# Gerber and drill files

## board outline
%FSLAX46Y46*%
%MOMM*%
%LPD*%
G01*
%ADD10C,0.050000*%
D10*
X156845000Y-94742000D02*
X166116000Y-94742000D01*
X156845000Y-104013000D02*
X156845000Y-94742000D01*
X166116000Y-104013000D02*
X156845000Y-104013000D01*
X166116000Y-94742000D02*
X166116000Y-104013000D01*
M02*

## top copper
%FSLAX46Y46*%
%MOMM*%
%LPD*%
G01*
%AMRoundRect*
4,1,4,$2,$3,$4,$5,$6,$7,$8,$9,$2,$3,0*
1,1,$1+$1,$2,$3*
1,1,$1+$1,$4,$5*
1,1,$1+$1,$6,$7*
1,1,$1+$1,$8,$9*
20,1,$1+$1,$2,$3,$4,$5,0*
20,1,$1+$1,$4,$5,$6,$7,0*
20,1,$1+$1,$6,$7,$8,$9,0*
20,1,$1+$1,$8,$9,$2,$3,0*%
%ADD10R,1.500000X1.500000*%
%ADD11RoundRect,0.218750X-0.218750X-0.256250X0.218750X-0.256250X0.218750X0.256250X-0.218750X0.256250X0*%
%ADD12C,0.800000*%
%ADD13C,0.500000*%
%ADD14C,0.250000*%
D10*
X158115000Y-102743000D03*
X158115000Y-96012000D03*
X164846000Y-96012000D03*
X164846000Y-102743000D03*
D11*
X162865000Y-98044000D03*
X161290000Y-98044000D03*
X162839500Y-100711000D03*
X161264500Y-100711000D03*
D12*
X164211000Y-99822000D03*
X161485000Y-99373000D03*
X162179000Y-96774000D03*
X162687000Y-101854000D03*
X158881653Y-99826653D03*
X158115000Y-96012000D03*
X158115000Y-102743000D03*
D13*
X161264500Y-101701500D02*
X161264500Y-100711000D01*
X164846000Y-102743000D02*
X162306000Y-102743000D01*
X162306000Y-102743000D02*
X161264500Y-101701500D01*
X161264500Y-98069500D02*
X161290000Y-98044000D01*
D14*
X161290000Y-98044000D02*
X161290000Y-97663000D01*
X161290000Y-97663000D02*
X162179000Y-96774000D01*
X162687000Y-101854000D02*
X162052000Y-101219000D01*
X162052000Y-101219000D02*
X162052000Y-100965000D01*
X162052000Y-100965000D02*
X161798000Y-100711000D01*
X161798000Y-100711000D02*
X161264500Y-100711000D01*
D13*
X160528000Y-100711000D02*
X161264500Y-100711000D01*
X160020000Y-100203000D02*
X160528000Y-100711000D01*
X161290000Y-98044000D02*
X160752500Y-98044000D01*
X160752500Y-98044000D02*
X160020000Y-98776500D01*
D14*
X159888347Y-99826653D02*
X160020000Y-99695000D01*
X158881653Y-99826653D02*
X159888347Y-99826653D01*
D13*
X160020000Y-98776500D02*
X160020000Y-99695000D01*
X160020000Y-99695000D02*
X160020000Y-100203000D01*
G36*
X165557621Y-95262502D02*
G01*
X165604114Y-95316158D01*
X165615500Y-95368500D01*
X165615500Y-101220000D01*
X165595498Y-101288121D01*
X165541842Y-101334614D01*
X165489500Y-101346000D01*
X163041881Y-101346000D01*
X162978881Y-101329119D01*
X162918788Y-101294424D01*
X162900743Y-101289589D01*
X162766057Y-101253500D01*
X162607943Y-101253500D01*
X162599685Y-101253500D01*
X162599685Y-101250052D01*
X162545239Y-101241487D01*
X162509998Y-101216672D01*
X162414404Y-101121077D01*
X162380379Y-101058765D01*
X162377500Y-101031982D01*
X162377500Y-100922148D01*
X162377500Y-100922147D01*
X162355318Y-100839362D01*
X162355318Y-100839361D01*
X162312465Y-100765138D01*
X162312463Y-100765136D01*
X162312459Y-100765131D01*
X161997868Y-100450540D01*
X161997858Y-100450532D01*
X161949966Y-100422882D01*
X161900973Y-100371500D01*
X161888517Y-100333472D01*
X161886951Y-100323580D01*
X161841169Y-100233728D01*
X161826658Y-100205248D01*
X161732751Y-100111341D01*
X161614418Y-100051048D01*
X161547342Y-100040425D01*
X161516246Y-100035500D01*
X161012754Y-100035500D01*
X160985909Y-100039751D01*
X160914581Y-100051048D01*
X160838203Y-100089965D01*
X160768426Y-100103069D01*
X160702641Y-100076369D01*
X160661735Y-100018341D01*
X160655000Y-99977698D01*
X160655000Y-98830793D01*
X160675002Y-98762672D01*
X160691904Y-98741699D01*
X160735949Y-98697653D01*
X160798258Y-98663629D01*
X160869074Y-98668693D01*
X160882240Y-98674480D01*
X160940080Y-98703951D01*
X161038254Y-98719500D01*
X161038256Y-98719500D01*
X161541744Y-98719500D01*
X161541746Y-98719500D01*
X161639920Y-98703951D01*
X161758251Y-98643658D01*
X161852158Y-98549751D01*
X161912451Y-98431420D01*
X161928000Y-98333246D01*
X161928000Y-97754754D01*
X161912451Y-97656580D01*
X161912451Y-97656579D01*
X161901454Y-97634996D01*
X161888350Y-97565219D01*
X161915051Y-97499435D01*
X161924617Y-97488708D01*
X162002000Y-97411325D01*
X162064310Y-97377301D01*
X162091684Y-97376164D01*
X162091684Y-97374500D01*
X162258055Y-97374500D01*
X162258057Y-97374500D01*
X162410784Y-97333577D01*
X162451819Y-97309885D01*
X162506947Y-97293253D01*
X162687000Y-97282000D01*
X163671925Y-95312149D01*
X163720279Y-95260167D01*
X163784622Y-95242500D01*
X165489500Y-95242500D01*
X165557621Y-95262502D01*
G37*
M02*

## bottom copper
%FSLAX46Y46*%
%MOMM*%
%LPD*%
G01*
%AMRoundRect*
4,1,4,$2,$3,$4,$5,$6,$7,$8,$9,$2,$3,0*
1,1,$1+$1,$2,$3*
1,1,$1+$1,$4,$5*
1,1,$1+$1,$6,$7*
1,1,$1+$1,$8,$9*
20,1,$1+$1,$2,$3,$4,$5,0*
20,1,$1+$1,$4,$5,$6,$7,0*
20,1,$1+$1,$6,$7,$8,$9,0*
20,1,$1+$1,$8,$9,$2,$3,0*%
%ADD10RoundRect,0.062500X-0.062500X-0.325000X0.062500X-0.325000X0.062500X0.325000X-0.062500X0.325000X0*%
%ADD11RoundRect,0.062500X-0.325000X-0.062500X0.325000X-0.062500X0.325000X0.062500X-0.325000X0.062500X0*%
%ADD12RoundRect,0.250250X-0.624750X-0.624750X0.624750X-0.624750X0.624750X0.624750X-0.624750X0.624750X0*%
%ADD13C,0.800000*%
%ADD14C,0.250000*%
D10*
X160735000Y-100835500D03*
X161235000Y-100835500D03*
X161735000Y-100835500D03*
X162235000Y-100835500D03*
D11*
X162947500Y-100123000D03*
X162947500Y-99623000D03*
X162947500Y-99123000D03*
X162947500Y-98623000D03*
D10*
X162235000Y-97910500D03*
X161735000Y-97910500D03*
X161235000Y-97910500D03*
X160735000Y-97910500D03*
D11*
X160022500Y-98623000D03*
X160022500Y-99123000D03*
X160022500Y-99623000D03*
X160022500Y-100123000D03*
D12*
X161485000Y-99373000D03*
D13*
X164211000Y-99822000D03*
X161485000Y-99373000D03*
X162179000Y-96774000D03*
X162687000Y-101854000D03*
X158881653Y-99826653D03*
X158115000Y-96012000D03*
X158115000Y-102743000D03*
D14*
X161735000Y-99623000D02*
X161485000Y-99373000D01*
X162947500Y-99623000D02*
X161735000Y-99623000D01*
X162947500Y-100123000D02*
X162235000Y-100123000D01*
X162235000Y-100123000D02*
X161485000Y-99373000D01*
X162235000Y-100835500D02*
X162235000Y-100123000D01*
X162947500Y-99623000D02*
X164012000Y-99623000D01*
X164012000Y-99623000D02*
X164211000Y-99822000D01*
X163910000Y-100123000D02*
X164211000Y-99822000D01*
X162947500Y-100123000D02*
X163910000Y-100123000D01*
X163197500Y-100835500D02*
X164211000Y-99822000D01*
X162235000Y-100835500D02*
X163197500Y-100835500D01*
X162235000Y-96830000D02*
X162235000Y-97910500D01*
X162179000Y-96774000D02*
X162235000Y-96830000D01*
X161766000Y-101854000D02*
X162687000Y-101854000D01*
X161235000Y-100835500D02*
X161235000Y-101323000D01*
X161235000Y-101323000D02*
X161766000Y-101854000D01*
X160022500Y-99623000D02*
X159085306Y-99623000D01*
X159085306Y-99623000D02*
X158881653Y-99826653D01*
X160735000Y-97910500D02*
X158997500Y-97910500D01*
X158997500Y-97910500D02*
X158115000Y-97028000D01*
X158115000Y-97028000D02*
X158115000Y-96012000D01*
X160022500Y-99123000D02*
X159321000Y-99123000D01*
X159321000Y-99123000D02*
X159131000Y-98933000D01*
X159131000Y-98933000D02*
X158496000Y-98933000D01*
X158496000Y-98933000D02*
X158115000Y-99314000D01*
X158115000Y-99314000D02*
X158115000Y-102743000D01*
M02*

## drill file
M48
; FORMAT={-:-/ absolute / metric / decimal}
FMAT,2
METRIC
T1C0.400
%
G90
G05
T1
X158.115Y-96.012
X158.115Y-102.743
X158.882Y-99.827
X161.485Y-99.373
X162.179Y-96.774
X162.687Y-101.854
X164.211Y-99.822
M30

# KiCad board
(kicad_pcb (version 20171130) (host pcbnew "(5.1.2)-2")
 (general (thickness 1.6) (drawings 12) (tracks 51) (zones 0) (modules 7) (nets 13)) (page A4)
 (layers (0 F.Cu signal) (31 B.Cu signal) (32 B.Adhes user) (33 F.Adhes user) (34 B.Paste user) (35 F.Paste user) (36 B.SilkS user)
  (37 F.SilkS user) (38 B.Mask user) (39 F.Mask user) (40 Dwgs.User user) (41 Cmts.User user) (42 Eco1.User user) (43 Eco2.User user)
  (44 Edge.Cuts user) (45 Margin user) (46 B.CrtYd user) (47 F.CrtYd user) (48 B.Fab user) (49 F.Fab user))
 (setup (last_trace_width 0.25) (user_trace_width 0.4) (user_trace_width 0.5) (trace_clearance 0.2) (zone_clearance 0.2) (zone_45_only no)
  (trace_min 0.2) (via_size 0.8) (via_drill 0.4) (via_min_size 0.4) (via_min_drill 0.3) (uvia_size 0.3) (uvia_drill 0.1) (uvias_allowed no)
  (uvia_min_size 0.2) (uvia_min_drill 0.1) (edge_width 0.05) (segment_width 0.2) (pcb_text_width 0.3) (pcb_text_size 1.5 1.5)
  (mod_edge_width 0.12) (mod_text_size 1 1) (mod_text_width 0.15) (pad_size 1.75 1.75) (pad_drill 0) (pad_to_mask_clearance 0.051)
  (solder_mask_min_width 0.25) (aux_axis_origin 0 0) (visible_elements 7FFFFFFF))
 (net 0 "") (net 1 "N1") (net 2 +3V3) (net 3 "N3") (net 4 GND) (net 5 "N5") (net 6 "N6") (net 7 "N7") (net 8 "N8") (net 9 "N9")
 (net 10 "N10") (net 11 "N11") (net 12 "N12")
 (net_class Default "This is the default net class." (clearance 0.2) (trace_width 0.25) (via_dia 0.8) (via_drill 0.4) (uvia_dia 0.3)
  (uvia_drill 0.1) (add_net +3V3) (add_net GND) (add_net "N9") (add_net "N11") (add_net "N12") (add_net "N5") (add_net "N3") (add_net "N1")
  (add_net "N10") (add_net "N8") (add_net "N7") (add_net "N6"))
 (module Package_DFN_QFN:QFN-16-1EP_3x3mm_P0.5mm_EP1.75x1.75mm (layer B.Cu) (at 161.485 99.373)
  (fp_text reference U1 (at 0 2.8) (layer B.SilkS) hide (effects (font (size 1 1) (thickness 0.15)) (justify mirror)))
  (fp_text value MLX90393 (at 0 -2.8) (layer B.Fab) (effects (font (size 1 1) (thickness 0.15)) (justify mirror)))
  (pad 16 smd roundrect (at -0.75 1.4625) (size 0.25 0.775) (layers B.Cu B.Paste B.Mask) (roundrect_rratio 0.25) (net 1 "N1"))
  (pad 15 smd roundrect (at -0.25 1.4625) (size 0.25 0.775) (layers B.Cu B.Paste B.Mask) (roundrect_rratio 0.25) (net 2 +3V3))
  (pad 14 smd roundrect (at 0.25 1.4625) (size 0.25 0.775) (layers B.Cu B.Paste B.Mask) (roundrect_rratio 0.25) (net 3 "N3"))
  (pad 13 smd roundrect (at 0.75 1.4625) (size 0.25 0.775) (layers B.Cu B.Paste B.Mask) (roundrect_rratio 0.25) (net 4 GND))
  (pad 12 smd roundrect (at 1.4625 0.75) (size 0.775 0.25) (layers B.Cu B.Paste B.Mask) (roundrect_rratio 0.25) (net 4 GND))
  (pad 11 smd roundrect (at 1.4625 0.25) (size 0.775 0.25) (layers B.Cu B.Paste B.Mask) (roundrect_rratio 0.25) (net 4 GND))
  (pad 10 smd roundrect (at 1.4625 -0.25) (size 0.775 0.25) (layers B.Cu B.Paste B.Mask) (roundrect_rratio 0.25) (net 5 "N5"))
  (pad 9 smd roundrect (at 1.4625 -0.75) (size 0.775 0.25) (layers B.Cu B.Paste B.Mask) (roundrect_rratio 0.25) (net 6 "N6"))
  (pad 8 smd roundrect (at 0.75 -1.4625) (size 0.25 0.775) (layers B.Cu B.Paste B.Mask) (roundrect_rratio 0.25) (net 2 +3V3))
  (pad 7 smd roundrect (at 0.25 -1.4625) (size 0.25 0.775) (layers B.Cu B.Paste B.Mask) (roundrect_rratio 0.25) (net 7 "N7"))
  (pad 6 smd roundrect (at -0.25 -1.4625) (size 0.25 0.775) (layers B.Cu B.Paste B.Mask) (roundrect_rratio 0.25) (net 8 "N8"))
  (pad 5 smd roundrect (at -0.75 -1.4625) (size 0.25 0.775) (layers B.Cu B.Paste B.Mask) (roundrect_rratio 0.25) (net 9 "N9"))
  (pad 4 smd roundrect (at -1.4625 -0.75) (size 0.775 0.25) (layers B.Cu B.Paste B.Mask) (roundrect_rratio 0.25) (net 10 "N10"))
  (pad 3 smd roundrect (at -1.4625 -0.25) (size 0.775 0.25) (layers B.Cu B.Paste B.Mask) (roundrect_rratio 0.25) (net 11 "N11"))
  (pad 2 smd roundrect (at -1.4625 0.25) (size 0.775 0.25) (layers B.Cu B.Paste B.Mask) (roundrect_rratio 0.25) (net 2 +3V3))
  (pad 1 smd roundrect (at -1.4625 0.75) (size 0.775 0.25) (layers B.Cu B.Paste B.Mask) (roundrect_rratio 0.25) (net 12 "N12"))
  (pad "" smd roundrect (at 0.44 -0.44) (size 0.71 0.71) (layers B.Paste) (roundrect_rratio 0.25))
  (pad "" smd roundrect (at 0.44 0.44) (size 0.71 0.71) (layers B.Paste) (roundrect_rratio 0.25))
  (pad "" smd roundrect (at -0.44 -0.44) (size 0.71 0.71) (layers B.Paste) (roundrect_rratio 0.25))
  (pad "" smd roundrect (at -0.44 0.44) (size 0.71 0.71) (layers B.Paste) (roundrect_rratio 0.25))
  (pad 17 smd roundrect (at 0 0) (size 1.75 1.75) (layers B.Cu B.Mask) (roundrect_rratio 0.143) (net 4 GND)))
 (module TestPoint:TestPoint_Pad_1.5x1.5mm (layer F.Cu) (at 158.115 102.743)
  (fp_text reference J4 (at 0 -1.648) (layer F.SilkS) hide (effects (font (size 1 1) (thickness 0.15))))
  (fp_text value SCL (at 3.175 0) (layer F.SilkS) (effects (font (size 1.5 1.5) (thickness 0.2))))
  (pad 1 smd rect (at 0 0) (size 1.5 1.5) (layers F.Cu F.Mask) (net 11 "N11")))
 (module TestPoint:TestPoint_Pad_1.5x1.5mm (layer F.Cu) (at 158.115 96.012)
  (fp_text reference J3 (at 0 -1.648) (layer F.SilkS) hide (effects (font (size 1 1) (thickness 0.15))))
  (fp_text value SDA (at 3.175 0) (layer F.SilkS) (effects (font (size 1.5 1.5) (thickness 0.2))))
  (pad 1 smd rect (at 0 0) (size 1.5 1.5) (layers F.Cu F.Mask) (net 9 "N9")))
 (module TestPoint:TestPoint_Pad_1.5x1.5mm (layer F.Cu) (at 164.846 96.012)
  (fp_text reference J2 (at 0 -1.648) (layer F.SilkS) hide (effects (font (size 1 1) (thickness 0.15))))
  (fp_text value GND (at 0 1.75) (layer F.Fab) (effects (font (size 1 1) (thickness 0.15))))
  (pad 1 smd rect (at 0 0) (size 1.5 1.5) (layers F.Cu F.Mask) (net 4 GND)))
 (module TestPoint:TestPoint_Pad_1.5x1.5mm (layer F.Cu) (at 164.846 102.743)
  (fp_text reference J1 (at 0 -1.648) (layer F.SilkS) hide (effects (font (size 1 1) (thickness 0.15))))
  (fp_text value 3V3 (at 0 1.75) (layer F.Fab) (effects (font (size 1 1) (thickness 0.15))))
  (pad 1 smd rect (at 0 0) (size 1.5 1.5) (layers F.Cu F.Mask) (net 2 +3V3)))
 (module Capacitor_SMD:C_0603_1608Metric (layer F.Cu) (at 162.0775 98.044)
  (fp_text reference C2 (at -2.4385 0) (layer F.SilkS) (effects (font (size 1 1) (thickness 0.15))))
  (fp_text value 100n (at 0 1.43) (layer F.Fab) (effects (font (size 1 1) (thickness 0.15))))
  (pad 2 smd roundrect (at 0.7875 0) (size 0.875 0.95) (layers F.Cu F.Paste F.Mask) (roundrect_rratio 0.25) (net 4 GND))
  (pad 1 smd roundrect (at -0.7875 0) (size 0.875 0.95) (layers F.Cu F.Paste F.Mask) (roundrect_rratio 0.25) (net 2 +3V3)))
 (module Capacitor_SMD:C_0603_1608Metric (layer F.Cu) (at 162.052 100.711)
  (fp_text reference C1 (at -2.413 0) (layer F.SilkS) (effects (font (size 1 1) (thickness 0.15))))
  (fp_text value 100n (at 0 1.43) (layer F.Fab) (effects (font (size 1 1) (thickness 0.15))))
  (pad 2 smd roundrect (at 0.7875 0) (size 0.875 0.95) (layers F.Cu F.Paste F.Mask) (roundrect_rratio 0.25) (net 4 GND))
  (pad 1 smd roundrect (at -0.7875 0) (size 0.875 0.95) (layers F.Cu F.Paste F.Mask) (roundrect_rratio 0.25) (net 2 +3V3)))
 (gr_line (start 156.845 94.742) (end 166.116 94.742) (layer Edge.Cuts) (width 0.05))
 (gr_line (start 156.845 104.013) (end 156.845 94.742) (layer Edge.Cuts) (width 0.05))
 (gr_line (start 166.116 104.013) (end 156.845 104.013) (layer Edge.Cuts) (width 0.05))
 (gr_line (start 166.116 94.742) (end 166.116 104.013) (layer Edge.Cuts) (width 0.05))
 (segment (start 161.735 99.623) (end 161.485 99.373) (width 0.25) (layer B.Cu) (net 4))
 (segment (start 162.9475 99.623) (end 161.735 99.623) (width 0.25) (layer B.Cu) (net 4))
 (segment (start 162.9475 100.123) (end 162.235 100.123) (width 0.25) (layer B.Cu) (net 4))
 (segment (start 162.235 100.123) (end 161.485 99.373) (width 0.25) (layer B.Cu) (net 4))
 (segment (start 162.235 100.8355) (end 162.235 100.123) (width 0.25) (layer B.Cu) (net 4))
 (via (at 164.211 99.822) (size 0.8) (drill 0.4) (layers F.Cu B.Cu) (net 4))
 (segment (start 162.9475 99.623) (end 164.012 99.623) (width 0.25) (layer B.Cu) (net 4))
 (segment (start 164.012 99.623) (end 164.211 99.822) (width 0.25) (layer B.Cu) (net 4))
 (segment (start 163.91 100.123) (end 164.211 99.822) (width 0.25) (layer B.Cu) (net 4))
 (segment (start 162.9475 100.123) (end 163.91 100.123) (width 0.25) (layer B.Cu) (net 4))
 (segment (start 163.1975 100.8355) (end 164.211 99.822) (width 0.25) (layer B.Cu) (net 4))
 (segment (start 162.235 100.8355) (end 163.1975 100.8355) (width 0.25) (layer B.Cu) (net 4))
 (via (at 161.485 99.373) (size 0.8) (drill 0.4) (layers F.Cu B.Cu) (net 4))
 (segment (start 161.2645 101.7015) (end 161.2645 100.711) (width 0.5) (layer F.Cu) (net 2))
 (segment (start 164.846 102.743) (end 162.306 102.743) (width 0.5) (layer F.Cu) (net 2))
 (segment (start 162.306 102.743) (end 161.2645 101.7015) (width 0.5) (layer F.Cu) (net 2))
 (segment (start 161.2645 98.0695) (end 161.29 98.044) (width 0.5) (layer F.Cu) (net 2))
 (via (at 162.179 96.774) (size 0.8) (drill 0.4) (layers F.Cu B.Cu) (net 2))
 (segment (start 161.29 98.044) (end 161.29 97.663) (width 0.25) (layer F.Cu) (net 2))
 (segment (start 161.29 97.663) (end 162.179 96.774) (width 0.25) (layer F.Cu) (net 2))
 (segment (start 162.235 96.83) (end 162.235 97.9105) (width 0.25) (layer B.Cu) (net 2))
 (segment (start 162.179 96.774) (end 162.235 96.83) (width 0.25) (layer B.Cu) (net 2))
 (via (at 162.687 101.854) (size 0.8) (drill 0.4) (layers F.Cu B.Cu) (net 2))
 (segment (start 161.766 101.854) (end 162.687 101.854) (width 0.25) (layer B.Cu) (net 2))
 (segment (start 161.235 100.8355) (end 161.235 101.323) (width 0.25) (layer B.Cu) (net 2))
 (segment (start 161.235 101.323) (end 161.766 101.854) (width 0.25) (layer B.Cu) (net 2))
 (segment (start 162.687 101.854) (end 162.052 101.219) (width 0.25) (layer F.Cu) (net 2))
 (segment (start 162.052 101.219) (end 162.052 100.965) (width 0.25) (layer F.Cu) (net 2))
 (segment (start 162.052 100.965) (end 161.798 100.711) (width 0.25) (layer F.Cu) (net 2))
 (segment (start 161.798 100.711) (end 161.2645 100.711) (width 0.25) (layer F.Cu) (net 2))
 (via (at 158.881653 99.826653) (size 0.8) (drill 0.4) (layers F.Cu B.Cu) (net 2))
 (segment (start 160.0225 99.623) (end 159.085306 99.623) (width 0.25) (layer B.Cu) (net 2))
 (segment (start 159.085306 99.623) (end 158.881653 99.826653) (width 0.25) (layer B.Cu) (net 2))
 (segment (start 160.528 100.711) (end 161.2645 100.711) (width 0.5) (layer F.Cu) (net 2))
 (segment (start 160.02 100.203) (end 160.528 100.711) (width 0.5) (layer F.Cu) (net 2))
 (segment (start 161.29 98.044) (end 160.7525 98.044) (width 0.5) (layer F.Cu) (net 2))
 (segment (start 160.7525 98.044) (end 160.02 98.7765) (width 0.5) (layer F.Cu) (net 2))
 (segment (start 159.888347 99.826653) (end 160.02 99.695) (width 0.25) (layer F.Cu) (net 2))
 (segment (start 158.881653 99.826653) (end 159.888347 99.826653) (width 0.25) (layer F.Cu) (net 2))
 (segment (start 160.02 98.7765) (end 160.02 99.695) (width 0.5) (layer F.Cu) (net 2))
 (segment (start 160.02 99.695) (end 160.02 100.203) (width 0.5) (layer F.Cu) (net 2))
 (segment (start 160.735 97.9105) (end 158.9975 97.9105) (width 0.25) (layer B.Cu) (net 9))
 (via (at 158.115 96.012) (size 0.8) (drill 0.4) (layers F.Cu B.Cu) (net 9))
 (segment (start 158.9975 97.9105) (end 158.115 97.028) (width 0.25) (layer B.Cu) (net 9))
 (segment (start 158.115 97.028) (end 158.115 96.012) (width 0.25) (layer B.Cu) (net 9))
 (segment (start 160.0225 99.123) (end 159.321 99.123) (width 0.25) (layer B.Cu) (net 11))
 (segment (start 159.321 99.123) (end 159.131 98.933) (width 0.25) (layer B.Cu) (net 11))
 (segment (start 159.131 98.933) (end 158.496 98.933) (width 0.25) (layer B.Cu) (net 11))
 (via (at 158.115 102.743) (size 0.8) (drill 0.4) (layers F.Cu B.Cu) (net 11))
 (segment (start 158.496 98.933) (end 158.115 99.314) (width 0.25) (layer B.Cu) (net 11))
 (segment (start 158.115 99.314) (end 158.115 102.743) (width 0.25) (layer B.Cu) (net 11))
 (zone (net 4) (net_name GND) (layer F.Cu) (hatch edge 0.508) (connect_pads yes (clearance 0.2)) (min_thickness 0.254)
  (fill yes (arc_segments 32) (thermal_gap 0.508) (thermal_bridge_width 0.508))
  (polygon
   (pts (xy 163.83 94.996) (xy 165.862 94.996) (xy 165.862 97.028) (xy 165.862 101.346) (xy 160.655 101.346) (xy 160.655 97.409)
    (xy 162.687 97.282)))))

